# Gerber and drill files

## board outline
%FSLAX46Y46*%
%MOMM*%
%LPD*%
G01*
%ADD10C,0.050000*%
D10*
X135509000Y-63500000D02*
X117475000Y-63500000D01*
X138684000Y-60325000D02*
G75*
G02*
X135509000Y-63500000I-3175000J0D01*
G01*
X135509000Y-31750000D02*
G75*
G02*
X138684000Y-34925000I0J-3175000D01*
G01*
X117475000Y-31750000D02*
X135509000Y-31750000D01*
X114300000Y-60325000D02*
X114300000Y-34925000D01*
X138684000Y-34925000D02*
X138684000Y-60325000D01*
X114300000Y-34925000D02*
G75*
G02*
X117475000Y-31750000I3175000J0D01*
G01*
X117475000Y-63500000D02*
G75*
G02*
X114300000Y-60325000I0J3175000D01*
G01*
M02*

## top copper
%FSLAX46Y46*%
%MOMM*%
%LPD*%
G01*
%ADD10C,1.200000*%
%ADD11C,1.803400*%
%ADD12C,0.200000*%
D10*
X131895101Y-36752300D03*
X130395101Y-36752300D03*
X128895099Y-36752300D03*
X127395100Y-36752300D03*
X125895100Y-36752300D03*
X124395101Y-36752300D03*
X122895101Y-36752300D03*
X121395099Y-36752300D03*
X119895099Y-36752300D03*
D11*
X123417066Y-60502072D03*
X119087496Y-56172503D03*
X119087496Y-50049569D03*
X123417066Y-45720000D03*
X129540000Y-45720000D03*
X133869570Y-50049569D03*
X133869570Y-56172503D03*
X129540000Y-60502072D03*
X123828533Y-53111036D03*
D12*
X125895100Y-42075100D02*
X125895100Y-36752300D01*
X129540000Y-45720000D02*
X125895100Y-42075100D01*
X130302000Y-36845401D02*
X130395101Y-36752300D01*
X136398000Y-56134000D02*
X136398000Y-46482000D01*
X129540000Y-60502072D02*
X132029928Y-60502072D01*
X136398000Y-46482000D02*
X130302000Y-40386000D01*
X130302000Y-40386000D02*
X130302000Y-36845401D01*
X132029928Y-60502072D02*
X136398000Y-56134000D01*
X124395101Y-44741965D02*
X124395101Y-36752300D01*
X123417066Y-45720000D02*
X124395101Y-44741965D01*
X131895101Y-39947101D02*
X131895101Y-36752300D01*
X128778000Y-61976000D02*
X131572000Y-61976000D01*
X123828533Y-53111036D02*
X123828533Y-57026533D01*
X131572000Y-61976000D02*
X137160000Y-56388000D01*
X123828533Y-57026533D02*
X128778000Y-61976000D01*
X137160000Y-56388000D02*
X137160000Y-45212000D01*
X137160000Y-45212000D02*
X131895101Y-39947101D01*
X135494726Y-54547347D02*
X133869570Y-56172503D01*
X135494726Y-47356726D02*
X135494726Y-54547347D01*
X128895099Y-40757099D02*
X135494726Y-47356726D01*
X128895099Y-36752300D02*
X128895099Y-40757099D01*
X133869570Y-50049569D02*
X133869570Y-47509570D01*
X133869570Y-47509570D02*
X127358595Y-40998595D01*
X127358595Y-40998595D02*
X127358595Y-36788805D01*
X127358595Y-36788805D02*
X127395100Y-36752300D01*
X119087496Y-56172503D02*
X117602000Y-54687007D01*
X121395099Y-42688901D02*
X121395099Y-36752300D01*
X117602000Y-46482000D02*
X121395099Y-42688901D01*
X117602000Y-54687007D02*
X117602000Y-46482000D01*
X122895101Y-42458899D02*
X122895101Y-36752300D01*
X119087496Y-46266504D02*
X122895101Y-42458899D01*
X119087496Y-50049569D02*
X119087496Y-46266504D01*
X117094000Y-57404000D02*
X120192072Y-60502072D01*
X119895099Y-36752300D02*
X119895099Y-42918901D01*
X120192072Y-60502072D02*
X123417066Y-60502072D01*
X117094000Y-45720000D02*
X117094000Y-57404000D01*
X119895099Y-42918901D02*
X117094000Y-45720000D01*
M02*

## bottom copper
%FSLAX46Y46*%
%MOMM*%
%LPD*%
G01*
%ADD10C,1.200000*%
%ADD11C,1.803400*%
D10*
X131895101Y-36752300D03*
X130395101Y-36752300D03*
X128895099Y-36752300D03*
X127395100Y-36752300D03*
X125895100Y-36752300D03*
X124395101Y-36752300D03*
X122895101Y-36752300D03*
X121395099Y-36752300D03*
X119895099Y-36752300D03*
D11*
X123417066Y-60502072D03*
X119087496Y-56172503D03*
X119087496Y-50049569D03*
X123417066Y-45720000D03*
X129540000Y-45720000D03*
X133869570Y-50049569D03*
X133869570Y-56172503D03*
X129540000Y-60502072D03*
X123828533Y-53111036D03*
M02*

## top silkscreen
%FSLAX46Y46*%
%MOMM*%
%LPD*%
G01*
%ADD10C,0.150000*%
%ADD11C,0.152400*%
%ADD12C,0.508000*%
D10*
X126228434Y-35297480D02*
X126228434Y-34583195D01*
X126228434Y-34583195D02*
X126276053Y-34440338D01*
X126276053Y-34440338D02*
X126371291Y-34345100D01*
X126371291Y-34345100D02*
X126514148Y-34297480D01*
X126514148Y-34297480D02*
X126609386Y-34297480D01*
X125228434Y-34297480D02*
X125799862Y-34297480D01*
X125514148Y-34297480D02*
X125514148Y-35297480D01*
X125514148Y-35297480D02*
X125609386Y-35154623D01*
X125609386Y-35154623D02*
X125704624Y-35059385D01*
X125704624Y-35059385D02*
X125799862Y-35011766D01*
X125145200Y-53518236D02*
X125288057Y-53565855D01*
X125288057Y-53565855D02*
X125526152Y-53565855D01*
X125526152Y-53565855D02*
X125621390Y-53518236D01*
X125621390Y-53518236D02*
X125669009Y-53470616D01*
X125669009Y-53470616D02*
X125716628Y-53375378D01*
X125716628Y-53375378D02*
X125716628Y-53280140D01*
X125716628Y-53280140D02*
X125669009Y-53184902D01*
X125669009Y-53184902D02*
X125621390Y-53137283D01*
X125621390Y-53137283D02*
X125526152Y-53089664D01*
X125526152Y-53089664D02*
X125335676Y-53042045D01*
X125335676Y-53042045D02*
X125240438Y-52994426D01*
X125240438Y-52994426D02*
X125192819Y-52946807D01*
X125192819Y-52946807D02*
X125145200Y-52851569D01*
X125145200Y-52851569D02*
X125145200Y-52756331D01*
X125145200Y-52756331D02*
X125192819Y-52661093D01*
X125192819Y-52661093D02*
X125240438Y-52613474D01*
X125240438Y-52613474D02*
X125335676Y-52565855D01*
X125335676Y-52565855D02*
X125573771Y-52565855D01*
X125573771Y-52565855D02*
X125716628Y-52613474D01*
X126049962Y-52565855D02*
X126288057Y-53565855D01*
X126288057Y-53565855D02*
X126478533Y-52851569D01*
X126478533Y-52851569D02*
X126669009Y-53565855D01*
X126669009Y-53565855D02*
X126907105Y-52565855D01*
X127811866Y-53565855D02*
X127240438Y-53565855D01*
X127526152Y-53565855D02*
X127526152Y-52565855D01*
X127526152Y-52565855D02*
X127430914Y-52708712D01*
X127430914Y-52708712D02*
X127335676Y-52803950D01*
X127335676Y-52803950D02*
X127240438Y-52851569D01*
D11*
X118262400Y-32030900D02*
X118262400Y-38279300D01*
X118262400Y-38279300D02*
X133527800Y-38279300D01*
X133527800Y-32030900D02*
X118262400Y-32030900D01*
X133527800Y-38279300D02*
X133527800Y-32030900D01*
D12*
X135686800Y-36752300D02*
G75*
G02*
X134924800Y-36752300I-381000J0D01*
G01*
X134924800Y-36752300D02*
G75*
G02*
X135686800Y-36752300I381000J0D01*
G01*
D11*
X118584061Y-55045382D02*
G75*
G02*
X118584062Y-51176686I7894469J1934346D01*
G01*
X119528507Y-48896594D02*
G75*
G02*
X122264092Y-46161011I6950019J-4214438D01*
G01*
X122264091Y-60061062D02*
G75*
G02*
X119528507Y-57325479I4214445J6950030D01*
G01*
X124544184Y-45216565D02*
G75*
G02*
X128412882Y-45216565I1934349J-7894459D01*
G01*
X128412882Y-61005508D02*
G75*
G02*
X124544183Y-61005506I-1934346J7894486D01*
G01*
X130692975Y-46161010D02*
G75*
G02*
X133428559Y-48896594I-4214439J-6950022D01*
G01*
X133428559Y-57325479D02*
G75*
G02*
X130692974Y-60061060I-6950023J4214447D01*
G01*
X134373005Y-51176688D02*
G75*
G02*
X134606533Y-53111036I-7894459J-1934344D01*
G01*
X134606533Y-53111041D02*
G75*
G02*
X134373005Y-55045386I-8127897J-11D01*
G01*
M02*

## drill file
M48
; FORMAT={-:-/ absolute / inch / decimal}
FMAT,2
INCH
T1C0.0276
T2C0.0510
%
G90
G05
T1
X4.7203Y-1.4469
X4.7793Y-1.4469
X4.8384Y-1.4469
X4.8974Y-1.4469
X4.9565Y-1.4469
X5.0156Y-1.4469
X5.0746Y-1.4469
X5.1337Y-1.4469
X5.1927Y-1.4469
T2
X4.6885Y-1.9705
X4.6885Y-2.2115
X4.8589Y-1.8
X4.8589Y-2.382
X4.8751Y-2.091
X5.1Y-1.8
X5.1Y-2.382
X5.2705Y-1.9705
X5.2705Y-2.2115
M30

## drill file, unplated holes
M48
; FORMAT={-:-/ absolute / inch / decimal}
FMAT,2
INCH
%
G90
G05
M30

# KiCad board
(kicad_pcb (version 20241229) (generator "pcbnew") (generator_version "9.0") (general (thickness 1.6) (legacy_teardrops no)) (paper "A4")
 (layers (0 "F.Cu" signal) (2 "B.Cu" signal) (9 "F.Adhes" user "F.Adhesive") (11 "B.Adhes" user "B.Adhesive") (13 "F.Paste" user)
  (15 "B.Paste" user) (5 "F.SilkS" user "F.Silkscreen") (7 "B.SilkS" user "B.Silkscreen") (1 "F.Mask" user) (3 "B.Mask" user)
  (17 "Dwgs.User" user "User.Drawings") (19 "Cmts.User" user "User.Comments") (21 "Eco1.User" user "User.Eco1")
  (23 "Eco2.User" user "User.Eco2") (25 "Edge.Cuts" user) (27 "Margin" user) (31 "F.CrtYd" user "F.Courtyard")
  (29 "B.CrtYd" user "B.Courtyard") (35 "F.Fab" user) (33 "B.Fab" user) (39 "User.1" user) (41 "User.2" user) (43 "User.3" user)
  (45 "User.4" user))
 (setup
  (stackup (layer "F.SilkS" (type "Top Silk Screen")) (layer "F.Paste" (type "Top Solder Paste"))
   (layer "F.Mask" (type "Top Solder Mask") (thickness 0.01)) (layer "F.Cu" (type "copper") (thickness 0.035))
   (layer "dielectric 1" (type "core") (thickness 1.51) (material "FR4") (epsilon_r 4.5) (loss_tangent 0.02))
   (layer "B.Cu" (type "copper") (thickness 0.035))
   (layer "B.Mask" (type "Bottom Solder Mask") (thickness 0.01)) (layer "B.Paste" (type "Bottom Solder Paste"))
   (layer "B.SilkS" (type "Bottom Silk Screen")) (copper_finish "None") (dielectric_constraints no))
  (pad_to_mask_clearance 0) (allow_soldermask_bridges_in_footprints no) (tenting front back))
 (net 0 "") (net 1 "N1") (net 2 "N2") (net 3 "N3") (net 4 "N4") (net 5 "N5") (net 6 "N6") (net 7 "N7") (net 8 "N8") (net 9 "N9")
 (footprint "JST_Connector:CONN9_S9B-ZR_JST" (layer "F.Cu") (at 131.895101 36.7523 180)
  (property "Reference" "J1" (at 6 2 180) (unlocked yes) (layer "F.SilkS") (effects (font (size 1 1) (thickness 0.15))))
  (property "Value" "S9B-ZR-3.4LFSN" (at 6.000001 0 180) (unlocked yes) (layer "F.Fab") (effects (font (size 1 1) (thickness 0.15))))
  (fp_line (start 13.632701 4.7214) (end 13.632701 -1.527) (stroke (width 0.1524) (type solid)) (layer "F.SilkS"))
  (fp_line (start 13.632701 -1.527) (end -1.632699 -1.527) (stroke (width 0.1524) (type solid)) (layer "F.SilkS"))
  (fp_line (start -1.632699 4.7214) (end 13.632701 4.7214) (stroke (width 0.1524) (type solid)) (layer "F.SilkS"))
  (fp_line (start -1.632699 -1.527) (end -1.632699 4.7214) (stroke (width 0.1524) (type solid)) (layer "F.SilkS"))
  (fp_circle (center -3.410699 0) (end -3.029699 0) (stroke (width 0.508) (type solid)) (fill no) (layer "F.SilkS"))
  (pad "1" thru_hole circle (at 0 0 180) (size 1.2 1.2) (drill 0.7) (layers "*.Cu" "*.Mask") (remove_unused_layers no) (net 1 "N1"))
  (pad "2" thru_hole circle (at 1.5 0 180) (size 1.2 1.2) (drill 0.7) (layers "*.Cu" "*.Mask") (remove_unused_layers no) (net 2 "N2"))
  (pad "3" thru_hole circle (at 3.000002 0 180) (size 1.2 1.2) (drill 0.7) (layers "*.Cu" "*.Mask") (remove_unused_layers no) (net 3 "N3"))
  (pad "4" thru_hole circle (at 4.500001 0 180) (size 1.2 1.2) (drill 0.7) (layers "*.Cu" "*.Mask") (remove_unused_layers no) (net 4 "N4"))
  (pad "5" thru_hole circle (at 6.000001 0 180) (size 1.2 1.2) (drill 0.7) (layers "*.Cu" "*.Mask") (remove_unused_layers no) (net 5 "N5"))
  (pad "6" thru_hole circle (at 7.5 0 180) (size 1.2 1.2) (drill 0.7) (layers "*.Cu" "*.Mask") (remove_unused_layers no) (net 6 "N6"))
  (pad "7" thru_hole circle (at 9 0 180) (size 1.2 1.2) (drill 0.7) (layers "*.Cu" "*.Mask") (remove_unused_layers no) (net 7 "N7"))
  (pad "8" thru_hole circle (at 10.500002 0 180) (size 1.2 1.2) (drill 0.7) (layers "*.Cu" "*.Mask") (remove_unused_layers no) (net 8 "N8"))
  (pad "9" thru_hole circle (at 12.000002 0 180) (size 1.2 1.2) (drill 0.7) (layers "*.Cu" "*.Mask") (remove_unused_layers no) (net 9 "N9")))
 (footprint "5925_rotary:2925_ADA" (layer "F.Cu") (at 123.417066 60.502072)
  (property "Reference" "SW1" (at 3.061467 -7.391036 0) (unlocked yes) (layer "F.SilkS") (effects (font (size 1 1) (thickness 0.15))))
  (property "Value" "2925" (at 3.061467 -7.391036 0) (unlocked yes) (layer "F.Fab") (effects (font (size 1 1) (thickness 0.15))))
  (fp_arc (start -4.833005 -5.45669) (mid -5.066533 -7.391038) (end -4.833004 -9.325386) (stroke (width 0.1524) (type solid))
   (layer "F.SilkS"))
  (fp_arc (start -3.888559 -11.605478) (mid -2.685897 -13.1384) (end -1.152975 -14.341062) (stroke (width 0.1524) (type solid))
   (layer "F.SilkS"))
  (fp_arc (start -1.152975 -0.44101) (mid -2.685897 -1.643672) (end -3.888559 -3.176593) (stroke (width 0.1524) (type solid))
   (layer "F.SilkS"))
  (fp_arc (start 1.127118 -15.285507) (mid 3.061467 -15.519036) (end 4.995816 -15.285507) (stroke (width 0.1524) (type solid))
   (layer "F.SilkS"))
  (fp_arc (start 4.995816 0.503436) (mid 3.061467 0.736964) (end 1.127117 0.503435) (stroke (width 0.1524) (type solid)) (layer "F.SilkS"))
  (fp_arc (start 7.275909 -14.341062) (mid 8.808831 -13.1384) (end 10.011493 -11.605478) (stroke (width 0.1524) (type solid))
   (layer "F.SilkS"))
  (fp_arc (start 10.011493 -3.176593) (mid 8.808831 -1.643672) (end 7.275909 -0.44101) (stroke (width 0.1524) (type solid))
   (layer "F.SilkS"))
  (fp_arc (start 10.955939 -9.325384) (mid 11.130874 -8.365233) (end 11.189467 -7.391036) (stroke (width 0.1524) (type solid))
   (layer "F.SilkS"))
  (fp_arc (start 11.189467 -7.391031) (mid 11.130874 -6.416836) (end 10.955938 -5.456686) (stroke (width 0.1524) (type solid))
   (layer "F.SilkS"))
  (pad "1" thru_hole circle (at 0 0) (size 1.8034 1.8034) (drill 1.2954) (layers "*.Cu" "*.Mask") (remove_unused_layers no) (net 9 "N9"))
  (pad "2" thru_hole circle (at -4.32957 -4.329569 315) (size 1.8034 1.8034) (drill 1.2954) (layers "*.Cu" "*.Mask")
   (remove_unused_layers no) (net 8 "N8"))
  (pad "3" thru_hole circle (at -4.32957 -10.452503 90) (size 1.8034 1.8034) (drill 1.2954) (layers "*.Cu" "*.Mask")
   (remove_unused_layers no) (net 7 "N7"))
  (pad "4" thru_hole circle (at 0 -14.782072 225) (size 1.8034 1.8034) (drill 1.2954) (layers "*.Cu" "*.Mask") (remove_unused_layers no)
   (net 6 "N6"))
  (pad "5" thru_hole circle (at 6.122934 -14.782072) (size 1.8034 1.8034) (drill 1.2954) (layers "*.Cu" "*.Mask") (remove_unused_layers no)
   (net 5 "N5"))
  (pad "6" thru_hole circle (at 10.452504 -10.452503 135) (size 1.8034 1.8034) (drill 1.2954) (layers "*.Cu" "*.Mask")
   (remove_unused_layers no) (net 4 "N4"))
  (pad "7" thru_hole circle (at 10.452504 -4.329569 90) (size 1.8034 1.8034) (drill 1.2954) (layers "*.Cu" "*.Mask")
   (remove_unused_layers no) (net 3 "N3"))
  (pad "8" thru_hole circle (at 6.122934 0 45) (size 1.8034 1.8034) (drill 1.2954) (layers "*.Cu" "*.Mask") (remove_unused_layers no)
   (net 2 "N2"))
  (pad "A" thru_hole circle (at 0.411467 -7.391036) (size 1.8034 1.8034) (drill 1.2954) (layers "*.Cu" "*.Mask") (remove_unused_layers no)
   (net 1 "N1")))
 (gr_line (start 135.509 63.5) (end 117.475 63.5) (stroke (width 0.05) (type default)) (layer "Edge.Cuts"))
 (gr_arc (start 138.684 60.325) (mid 137.754064 62.570064) (end 135.509 63.5) (stroke (width 0.05) (type default)) (layer "Edge.Cuts"))
 (gr_arc (start 135.509 31.75) (mid 137.754064 32.679936) (end 138.684 34.925) (stroke (width 0.05) (type default)) (layer "Edge.Cuts"))
 (gr_line (start 117.475 31.75) (end 135.509 31.75) (stroke (width 0.05) (type default)) (layer "Edge.Cuts"))
 (gr_line (start 114.3 60.325) (end 114.3 34.925) (stroke (width 0.05) (type default)) (layer "Edge.Cuts"))
 (gr_line (start 138.684 34.925) (end 138.684 60.325) (stroke (width 0.05) (type default)) (layer "Edge.Cuts"))
 (gr_arc (start 114.3 34.925) (mid 115.229936 32.679936) (end 117.475 31.75) (stroke (width 0.05) (type default)) (layer "Edge.Cuts"))
 (gr_arc (start 117.475 63.5) (mid 115.229936 62.570064) (end 114.3 60.325) (stroke (width 0.05) (type default)) (layer "Edge.Cuts"))
 (segment (start 125.8951 42.0751) (end 125.8951 36.7523) (width 0.2) (layer "F.Cu") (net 5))
 (segment (start 129.54 45.72) (end 125.8951 42.0751) (width 0.2) (layer "F.Cu") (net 5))
 (segment (start 130.302 36.845401) (end 130.395101 36.7523) (width 0.2) (layer "F.Cu") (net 2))
 (segment (start 136.398 56.134) (end 136.398 46.482) (width 0.2) (layer "F.Cu") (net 2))
 (segment (start 129.54 60.502072) (end 132.029928 60.502072) (width 0.2) (layer "F.Cu") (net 2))
 (segment (start 136.398 46.482) (end 130.302 40.386) (width 0.2) (layer "F.Cu") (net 2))
 (segment (start 130.302 40.386) (end 130.302 36.845401) (width 0.2) (layer "F.Cu") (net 2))
 (segment (start 132.029928 60.502072) (end 136.398 56.134) (width 0.2) (layer "F.Cu") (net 2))
 (segment (start 124.395101 44.741965) (end 124.395101 36.7523) (width 0.2) (layer "F.Cu") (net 6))
 (segment (start 123.417066 45.72) (end 124.395101 44.741965) (width 0.2) (layer "F.Cu") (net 6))
 (segment (start 131.895101 39.947101) (end 131.895101 36.7523) (width 0.2) (layer "F.Cu") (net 1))
 (segment (start 128.778 61.976) (end 131.572 61.976) (width 0.2) (layer "F.Cu") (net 1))
 (segment (start 123.828533 53.111036) (end 123.828533 57.026533) (width 0.2) (layer "F.Cu") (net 1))
 (segment (start 131.572 61.976) (end 137.16 56.388) (width 0.2) (layer "F.Cu") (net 1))
 (segment (start 123.828533 57.026533) (end 128.778 61.976) (width 0.2) (layer "F.Cu") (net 1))
 (segment (start 137.16 56.388) (end 137.16 45.212) (width 0.2) (layer "F.Cu") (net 1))
 (segment (start 137.16 45.212) (end 131.895101 39.947101) (width 0.2) (layer "F.Cu") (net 1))
 (segment (start 135.494726 54.547347) (end 133.86957 56.172503) (width 0.2) (layer "F.Cu") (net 3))
 (segment (start 135.494726 47.356726) (end 135.494726 54.547347) (width 0.2) (layer "F.Cu") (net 3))
 (segment (start 128.895099 40.757099) (end 135.494726 47.356726) (width 0.2) (layer "F.Cu") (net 3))
 (segment (start 128.895099 36.7523) (end 128.895099 40.757099) (width 0.2) (layer "F.Cu") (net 3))
 (segment (start 133.86957 50.049569) (end 133.86957 47.50957) (width 0.2) (layer "F.Cu") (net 4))
 (segment (start 133.86957 47.50957) (end 127.358595 40.998595) (width 0.2) (layer "F.Cu") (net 4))
 (segment (start 127.358595 40.998595) (end 127.358595 36.788805) (width 0.2) (layer "F.Cu") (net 4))
 (segment (start 127.358595 36.788805) (end 127.3951 36.7523) (width 0.2) (layer "F.Cu") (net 4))
 (segment (start 119.087496 56.172503) (end 117.602 54.687007) (width 0.2) (layer "F.Cu") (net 8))
 (segment (start 121.395099 42.688901) (end 121.395099 36.7523) (width 0.2) (layer "F.Cu") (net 8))
 (segment (start 117.602 46.482) (end 121.395099 42.688901) (width 0.2) (layer "F.Cu") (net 8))
 (segment (start 117.602 54.687007) (end 117.602 46.482) (width 0.2) (layer "F.Cu") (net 8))
 (segment (start 122.895101 42.458899) (end 122.895101 36.7523) (width 0.2) (layer "F.Cu") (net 7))
 (segment (start 119.087496 46.266504) (end 122.895101 42.458899) (width 0.2) (layer "F.Cu") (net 7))
 (segment (start 119.087496 50.049569) (end 119.087496 46.266504) (width 0.2) (layer "F.Cu") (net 7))
 (segment (start 117.094 57.404) (end 120.192072 60.502072) (width 0.2) (layer "F.Cu") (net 9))
 (segment (start 119.895099 36.7523) (end 119.895099 42.918901) (width 0.2) (layer "F.Cu") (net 9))
 (segment (start 120.192072 60.502072) (end 123.417066 60.502072) (width 0.2) (layer "F.Cu") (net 9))
 (segment (start 117.094 45.72) (end 117.094 57.404) (width 0.2) (layer "F.Cu") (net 9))
 (segment (start 119.895099 42.918901) (end 117.094 45.72) (width 0.2) (layer "F.Cu") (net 9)))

